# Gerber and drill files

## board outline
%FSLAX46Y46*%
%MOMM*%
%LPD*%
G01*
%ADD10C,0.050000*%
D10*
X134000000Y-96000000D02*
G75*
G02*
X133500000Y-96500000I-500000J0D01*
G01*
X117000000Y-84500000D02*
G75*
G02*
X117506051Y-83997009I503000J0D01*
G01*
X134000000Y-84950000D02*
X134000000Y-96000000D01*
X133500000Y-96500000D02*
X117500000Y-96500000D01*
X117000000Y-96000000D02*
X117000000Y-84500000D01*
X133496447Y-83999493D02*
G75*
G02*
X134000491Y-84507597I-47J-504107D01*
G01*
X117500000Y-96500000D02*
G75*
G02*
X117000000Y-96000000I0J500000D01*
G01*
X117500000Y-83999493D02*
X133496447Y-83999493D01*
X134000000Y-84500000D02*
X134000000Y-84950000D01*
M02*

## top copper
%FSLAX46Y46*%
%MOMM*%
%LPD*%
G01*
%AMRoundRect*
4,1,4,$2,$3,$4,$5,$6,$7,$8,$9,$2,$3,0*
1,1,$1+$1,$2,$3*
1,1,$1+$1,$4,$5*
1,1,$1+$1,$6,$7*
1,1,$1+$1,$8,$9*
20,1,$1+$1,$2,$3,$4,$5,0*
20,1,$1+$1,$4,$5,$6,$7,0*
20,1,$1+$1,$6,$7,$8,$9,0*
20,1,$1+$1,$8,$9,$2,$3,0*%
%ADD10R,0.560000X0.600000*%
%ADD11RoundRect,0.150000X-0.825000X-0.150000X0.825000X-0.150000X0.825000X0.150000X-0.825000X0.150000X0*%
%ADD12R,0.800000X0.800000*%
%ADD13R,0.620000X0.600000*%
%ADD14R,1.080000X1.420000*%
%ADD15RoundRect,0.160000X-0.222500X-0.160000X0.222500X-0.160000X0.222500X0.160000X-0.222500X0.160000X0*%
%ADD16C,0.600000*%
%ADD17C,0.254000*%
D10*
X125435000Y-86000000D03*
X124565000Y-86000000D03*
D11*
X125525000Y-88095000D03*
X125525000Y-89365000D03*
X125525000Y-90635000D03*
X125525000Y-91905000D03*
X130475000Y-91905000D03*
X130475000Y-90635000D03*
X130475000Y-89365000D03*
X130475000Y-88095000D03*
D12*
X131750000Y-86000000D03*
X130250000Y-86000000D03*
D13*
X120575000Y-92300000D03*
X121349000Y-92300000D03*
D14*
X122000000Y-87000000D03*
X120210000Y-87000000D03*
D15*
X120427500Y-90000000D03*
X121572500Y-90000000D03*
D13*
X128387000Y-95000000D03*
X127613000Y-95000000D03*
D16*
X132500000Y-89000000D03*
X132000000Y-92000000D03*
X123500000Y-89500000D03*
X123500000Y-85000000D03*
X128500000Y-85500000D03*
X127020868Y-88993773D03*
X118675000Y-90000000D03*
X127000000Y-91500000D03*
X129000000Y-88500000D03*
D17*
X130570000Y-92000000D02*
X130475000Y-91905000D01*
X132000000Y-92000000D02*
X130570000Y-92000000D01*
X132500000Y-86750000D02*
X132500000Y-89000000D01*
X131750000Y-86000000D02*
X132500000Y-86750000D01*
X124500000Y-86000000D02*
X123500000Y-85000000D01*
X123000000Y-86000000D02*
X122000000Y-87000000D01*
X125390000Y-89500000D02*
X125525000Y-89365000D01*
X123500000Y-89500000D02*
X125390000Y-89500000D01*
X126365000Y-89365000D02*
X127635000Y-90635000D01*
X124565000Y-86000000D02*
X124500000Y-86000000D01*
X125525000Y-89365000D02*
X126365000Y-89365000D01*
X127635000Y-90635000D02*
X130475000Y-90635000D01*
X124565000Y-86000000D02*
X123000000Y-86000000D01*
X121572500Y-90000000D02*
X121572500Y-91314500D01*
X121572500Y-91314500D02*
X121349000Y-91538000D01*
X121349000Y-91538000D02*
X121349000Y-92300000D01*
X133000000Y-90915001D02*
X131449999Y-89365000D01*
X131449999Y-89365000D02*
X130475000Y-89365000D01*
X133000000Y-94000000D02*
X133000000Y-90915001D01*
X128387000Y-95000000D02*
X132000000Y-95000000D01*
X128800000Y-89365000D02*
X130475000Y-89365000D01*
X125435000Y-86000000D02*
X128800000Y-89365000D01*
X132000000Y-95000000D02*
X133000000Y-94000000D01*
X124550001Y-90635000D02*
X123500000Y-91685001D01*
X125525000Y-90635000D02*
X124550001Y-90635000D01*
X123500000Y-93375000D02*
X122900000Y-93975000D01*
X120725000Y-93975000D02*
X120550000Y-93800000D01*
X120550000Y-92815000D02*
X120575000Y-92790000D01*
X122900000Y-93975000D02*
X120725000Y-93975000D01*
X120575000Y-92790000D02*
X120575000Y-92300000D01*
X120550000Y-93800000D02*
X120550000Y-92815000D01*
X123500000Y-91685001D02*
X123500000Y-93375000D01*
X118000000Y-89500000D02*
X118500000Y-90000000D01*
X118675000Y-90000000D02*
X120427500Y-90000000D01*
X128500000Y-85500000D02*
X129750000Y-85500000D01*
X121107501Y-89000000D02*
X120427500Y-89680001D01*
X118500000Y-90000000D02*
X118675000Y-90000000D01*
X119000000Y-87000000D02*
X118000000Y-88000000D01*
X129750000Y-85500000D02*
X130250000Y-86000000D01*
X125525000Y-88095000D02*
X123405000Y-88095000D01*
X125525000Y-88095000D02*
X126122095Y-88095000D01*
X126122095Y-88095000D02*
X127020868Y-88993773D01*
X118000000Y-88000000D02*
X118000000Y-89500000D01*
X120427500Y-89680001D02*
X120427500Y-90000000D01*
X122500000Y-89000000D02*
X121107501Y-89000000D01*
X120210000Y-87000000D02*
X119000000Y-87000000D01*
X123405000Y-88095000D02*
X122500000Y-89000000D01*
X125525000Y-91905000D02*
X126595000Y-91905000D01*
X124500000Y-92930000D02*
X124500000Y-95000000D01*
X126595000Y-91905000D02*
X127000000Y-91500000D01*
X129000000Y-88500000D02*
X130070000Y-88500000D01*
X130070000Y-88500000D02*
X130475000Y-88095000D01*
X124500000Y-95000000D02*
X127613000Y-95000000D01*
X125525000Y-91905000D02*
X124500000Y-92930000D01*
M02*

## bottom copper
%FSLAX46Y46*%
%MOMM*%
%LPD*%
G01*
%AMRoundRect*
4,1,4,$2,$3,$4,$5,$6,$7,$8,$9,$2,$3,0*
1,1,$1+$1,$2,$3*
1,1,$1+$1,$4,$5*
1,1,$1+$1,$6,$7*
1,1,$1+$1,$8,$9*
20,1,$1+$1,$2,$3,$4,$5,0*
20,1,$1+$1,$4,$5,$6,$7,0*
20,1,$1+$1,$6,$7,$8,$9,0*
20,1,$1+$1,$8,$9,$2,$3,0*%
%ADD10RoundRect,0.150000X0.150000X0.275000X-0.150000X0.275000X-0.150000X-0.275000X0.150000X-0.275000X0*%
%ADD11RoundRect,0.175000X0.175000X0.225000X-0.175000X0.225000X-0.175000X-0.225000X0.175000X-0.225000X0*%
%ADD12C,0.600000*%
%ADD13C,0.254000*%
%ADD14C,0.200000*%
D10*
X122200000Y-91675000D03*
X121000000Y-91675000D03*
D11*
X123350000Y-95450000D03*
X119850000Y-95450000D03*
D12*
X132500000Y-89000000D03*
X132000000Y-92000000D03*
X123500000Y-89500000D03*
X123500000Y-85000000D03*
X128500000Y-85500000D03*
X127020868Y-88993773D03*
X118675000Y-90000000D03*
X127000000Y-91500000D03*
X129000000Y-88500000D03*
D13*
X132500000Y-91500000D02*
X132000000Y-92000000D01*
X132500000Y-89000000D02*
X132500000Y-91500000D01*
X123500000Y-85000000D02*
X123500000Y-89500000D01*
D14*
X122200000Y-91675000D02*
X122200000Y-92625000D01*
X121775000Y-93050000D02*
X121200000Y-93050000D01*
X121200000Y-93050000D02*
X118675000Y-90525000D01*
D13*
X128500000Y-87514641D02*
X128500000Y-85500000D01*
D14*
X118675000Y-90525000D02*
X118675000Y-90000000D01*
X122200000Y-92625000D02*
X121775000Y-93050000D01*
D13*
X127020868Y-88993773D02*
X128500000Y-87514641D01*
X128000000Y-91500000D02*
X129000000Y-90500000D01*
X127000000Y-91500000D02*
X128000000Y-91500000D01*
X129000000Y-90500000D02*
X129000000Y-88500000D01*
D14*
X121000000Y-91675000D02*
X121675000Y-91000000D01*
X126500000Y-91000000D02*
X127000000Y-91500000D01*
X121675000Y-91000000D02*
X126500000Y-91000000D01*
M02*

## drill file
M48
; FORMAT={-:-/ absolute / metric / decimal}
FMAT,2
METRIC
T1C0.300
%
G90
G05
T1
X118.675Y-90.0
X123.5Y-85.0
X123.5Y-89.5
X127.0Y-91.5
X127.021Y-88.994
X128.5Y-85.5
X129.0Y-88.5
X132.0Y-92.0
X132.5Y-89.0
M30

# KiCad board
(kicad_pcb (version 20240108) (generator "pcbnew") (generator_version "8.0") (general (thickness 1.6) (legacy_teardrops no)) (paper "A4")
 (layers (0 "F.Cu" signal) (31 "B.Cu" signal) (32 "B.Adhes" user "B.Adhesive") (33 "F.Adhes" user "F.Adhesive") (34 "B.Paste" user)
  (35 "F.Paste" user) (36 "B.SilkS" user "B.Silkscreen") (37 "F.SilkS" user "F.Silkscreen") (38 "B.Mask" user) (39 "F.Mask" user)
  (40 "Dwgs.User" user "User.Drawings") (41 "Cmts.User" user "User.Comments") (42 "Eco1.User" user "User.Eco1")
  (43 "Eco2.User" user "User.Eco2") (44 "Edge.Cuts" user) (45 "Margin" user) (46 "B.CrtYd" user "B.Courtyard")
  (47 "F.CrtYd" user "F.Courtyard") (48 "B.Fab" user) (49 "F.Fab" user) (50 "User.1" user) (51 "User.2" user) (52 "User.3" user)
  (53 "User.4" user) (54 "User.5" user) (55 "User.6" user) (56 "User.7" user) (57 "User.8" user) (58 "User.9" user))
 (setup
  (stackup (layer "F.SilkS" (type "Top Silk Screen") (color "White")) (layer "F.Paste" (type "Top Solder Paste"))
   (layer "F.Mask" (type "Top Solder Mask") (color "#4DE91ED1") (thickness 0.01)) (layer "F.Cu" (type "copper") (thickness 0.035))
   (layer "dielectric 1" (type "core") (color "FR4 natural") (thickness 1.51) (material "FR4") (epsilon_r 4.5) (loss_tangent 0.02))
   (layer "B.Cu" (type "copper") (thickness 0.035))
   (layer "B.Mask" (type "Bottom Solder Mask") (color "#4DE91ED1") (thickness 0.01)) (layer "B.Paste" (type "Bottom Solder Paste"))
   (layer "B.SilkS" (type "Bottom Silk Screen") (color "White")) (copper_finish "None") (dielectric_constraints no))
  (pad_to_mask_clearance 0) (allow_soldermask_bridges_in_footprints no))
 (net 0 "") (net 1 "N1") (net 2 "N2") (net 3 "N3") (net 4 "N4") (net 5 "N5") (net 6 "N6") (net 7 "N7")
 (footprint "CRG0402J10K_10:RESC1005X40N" (layer "F.Cu") (at 125 86 180)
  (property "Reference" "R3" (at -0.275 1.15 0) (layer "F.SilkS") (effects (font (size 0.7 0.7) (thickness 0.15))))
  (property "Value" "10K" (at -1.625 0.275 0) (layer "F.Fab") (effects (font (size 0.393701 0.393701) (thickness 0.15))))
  (pad "1" smd rect (at -0.435 0 180) (size 0.56 0.6) (layers "F.Cu" "F.Paste" "F.Mask") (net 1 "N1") (solder_mask_margin 0.102))
  (pad "2" smd rect (at 0.435 0 180) (size 0.56 0.6) (layers "F.Cu" "F.Paste" "F.Mask") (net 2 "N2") (solder_mask_margin 0.102)))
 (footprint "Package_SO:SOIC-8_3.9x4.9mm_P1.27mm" (layer "F.Cu") (at 128 90)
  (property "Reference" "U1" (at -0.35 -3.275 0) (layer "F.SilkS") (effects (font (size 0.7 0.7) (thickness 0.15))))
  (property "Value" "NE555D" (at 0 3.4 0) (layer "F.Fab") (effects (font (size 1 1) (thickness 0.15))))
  (pad "1" smd roundrect (at -2.475 -1.905) (size 1.95 0.6) (layers "F.Cu" "F.Paste" "F.Mask") (roundrect_rratio 0.25) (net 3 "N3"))
  (pad "2" smd roundrect (at -2.475 -0.635) (size 1.95 0.6) (layers "F.Cu" "F.Paste" "F.Mask") (roundrect_rratio 0.25) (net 2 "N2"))
  (pad "3" smd roundrect (at -2.475 0.635) (size 1.95 0.6) (layers "F.Cu" "F.Paste" "F.Mask") (roundrect_rratio 0.25) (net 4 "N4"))
  (pad "4" smd roundrect (at -2.475 1.905) (size 1.95 0.6) (layers "F.Cu" "F.Paste" "F.Mask") (roundrect_rratio 0.25) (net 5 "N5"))
  (pad "5" smd roundrect (at 2.475 1.905) (size 1.95 0.6) (layers "F.Cu" "F.Paste" "F.Mask") (roundrect_rratio 0.25) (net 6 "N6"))
  (pad "6" smd roundrect (at 2.475 0.635) (size 1.95 0.6) (layers "F.Cu" "F.Paste" "F.Mask") (roundrect_rratio 0.25) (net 2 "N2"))
  (pad "7" smd roundrect (at 2.475 -0.635) (size 1.95 0.6) (layers "F.Cu" "F.Paste" "F.Mask") (roundrect_rratio 0.25) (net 1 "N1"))
  (pad "8" smd roundrect (at 2.475 -1.905) (size 1.95 0.6) (layers "F.Cu" "F.Paste" "F.Mask") (roundrect_rratio 0.25) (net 5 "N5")))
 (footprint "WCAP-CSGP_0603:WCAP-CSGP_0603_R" (layer "F.Cu") (at 131 86 180)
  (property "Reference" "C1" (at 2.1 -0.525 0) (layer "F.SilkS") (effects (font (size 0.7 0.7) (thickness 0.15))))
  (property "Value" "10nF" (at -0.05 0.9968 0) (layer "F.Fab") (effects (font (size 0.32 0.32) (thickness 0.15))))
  (pad "1" smd rect (at -0.75 0 180) (size 0.8 0.8) (layers "F.Cu" "F.Paste" "F.Mask") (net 6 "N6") (solder_mask_margin 0.102))
  (pad "2" smd rect (at 0.75 0 180) (size 0.8 0.8) (layers "F.Cu" "F.Paste" "F.Mask") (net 3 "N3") (solder_mask_margin 0.102)))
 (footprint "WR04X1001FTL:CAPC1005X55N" (layer "F.Cu") (at 120.962 92.3)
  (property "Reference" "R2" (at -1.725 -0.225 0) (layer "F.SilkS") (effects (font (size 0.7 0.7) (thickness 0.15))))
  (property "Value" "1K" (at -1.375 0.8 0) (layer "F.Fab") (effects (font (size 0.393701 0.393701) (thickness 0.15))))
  (pad "1" smd rect (at -0.387 0) (size 0.62 0.6) (layers "F.Cu" "F.Paste" "F.Mask") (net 4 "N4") (solder_mask_margin 0.05))
  (pad "2" smd rect (at 0.387 0) (size 0.62 0.6) (layers "F.Cu" "F.Paste" "F.Mask") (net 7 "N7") (solder_mask_margin 0.05)))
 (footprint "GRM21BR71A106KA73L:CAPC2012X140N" (layer "F.Cu") (at 121.105 87 180)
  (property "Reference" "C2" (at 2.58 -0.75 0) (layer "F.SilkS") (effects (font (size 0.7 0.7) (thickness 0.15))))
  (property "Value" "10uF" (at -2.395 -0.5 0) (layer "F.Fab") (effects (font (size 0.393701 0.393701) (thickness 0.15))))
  (pad "1" smd rect (at -0.895 0 180) (size 1.08 1.42) (layers "F.Cu" "F.Paste" "F.Mask") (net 2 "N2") (solder_mask_margin 0.102))
  (pad "2" smd rect (at 0.895 0 180) (size 1.08 1.42) (layers "F.Cu" "F.Paste" "F.Mask") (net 3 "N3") (solder_mask_margin 0.102)))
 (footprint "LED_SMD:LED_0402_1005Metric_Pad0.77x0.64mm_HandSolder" (layer "F.Cu") (at 121 90)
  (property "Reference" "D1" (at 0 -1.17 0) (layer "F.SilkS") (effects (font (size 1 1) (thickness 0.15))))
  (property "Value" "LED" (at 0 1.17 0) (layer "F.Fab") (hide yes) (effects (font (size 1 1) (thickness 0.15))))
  (pad "1" smd roundrect (at -0.5725 0) (size 0.765 0.64) (layers "F.Cu" "F.Paste" "F.Mask") (roundrect_rratio 0.25) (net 3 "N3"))
  (pad "2" smd roundrect (at 0.5725 0) (size 0.765 0.64) (layers "F.Cu" "F.Paste" "F.Mask") (roundrect_rratio 0.25) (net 7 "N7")))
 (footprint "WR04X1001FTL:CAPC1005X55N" (layer "F.Cu") (at 128 95 180)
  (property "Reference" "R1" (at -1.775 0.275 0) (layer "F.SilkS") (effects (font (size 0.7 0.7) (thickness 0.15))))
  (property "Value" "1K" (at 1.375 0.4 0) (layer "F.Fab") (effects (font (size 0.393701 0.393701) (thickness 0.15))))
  (pad "1" smd rect (at -0.387 0 180) (size 0.62 0.6) (layers "F.Cu" "F.Paste" "F.Mask") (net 1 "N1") (solder_mask_margin 0.05))
  (pad "2" smd rect (at 0.387 0 180) (size 0.62 0.6) (layers "F.Cu" "F.Paste" "F.Mask") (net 5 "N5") (solder_mask_margin 0.05)
   (teardrops (best_length_ratio 2) (max_length 1) (best_width_ratio 1) (max_width 2) (curve_points 0) (filter_ratio 0.9) (enabled no)
    (allow_two_segments yes) (prefer_zone_connections yes))))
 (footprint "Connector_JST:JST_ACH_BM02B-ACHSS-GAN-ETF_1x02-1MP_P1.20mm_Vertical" (layer "B.Cu") (at 121.6 93.55 180)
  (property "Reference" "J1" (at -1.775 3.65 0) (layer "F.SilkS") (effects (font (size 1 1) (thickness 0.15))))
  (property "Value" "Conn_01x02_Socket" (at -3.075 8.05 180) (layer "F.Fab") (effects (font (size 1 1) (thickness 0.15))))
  (pad "1" smd roundrect (at -0.6 1.875 180) (size 0.6 0.85) (layers "B.Cu" "B.Paste" "B.Mask") (roundrect_rratio 0.25) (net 3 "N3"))
  (pad "2" smd roundrect (at 0.6 1.875 180) (size 0.6 0.85) (layers "B.Cu" "B.Paste" "B.Mask") (roundrect_rratio 0.25) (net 5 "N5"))
  (pad "MP" smd roundrect (at -1.75 -1.9 180) (size 0.7 0.8) (layers "B.Cu" "B.Paste" "B.Mask") (roundrect_rratio 0.25))
  (pad "MP" smd roundrect (at 1.75 -1.9 180) (size 0.7 0.8) (layers "B.Cu" "B.Paste" "B.Mask") (roundrect_rratio 0.25)))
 (gr_arc (start 134 96) (mid 133.853553 96.353553) (end 133.5 96.5) (stroke (width 0.05) (type default)) (layer "Edge.Cuts"))
 (gr_arc (start 117 84.5) (mid 117.148404 84.143238) (end 117.506051 83.996979) (stroke (width 0.05) (type default)) (layer "Edge.Cuts"))
 (gr_line (start 134 84.95) (end 134 96) (stroke (width 0.05) (type default)) (layer "Edge.Cuts"))
 (gr_line (start 133.5 96.5) (end 117.5 96.5) (stroke (width 0.05) (type default)) (layer "Edge.Cuts"))
 (gr_line (start 117 96) (end 117 84.5) (stroke (width 0.05) (type default)) (layer "Edge.Cuts"))
 (gr_arc (start 133.496447 83.999493) (mid 133.854298 84.148562) (end 134.000491 84.507597) (stroke (width 0.05) (type default))
  (layer "Edge.Cuts"))
 (gr_arc (start 117.5 96.5) (mid 117.146447 96.353553) (end 117 96) (stroke (width 0.05) (type default)) (layer "Edge.Cuts"))
 (gr_line (start 117.5 83.999493) (end 133.496447 83.999493) (stroke (width 0.05) (type default)) (layer "Edge.Cuts"))
 (gr_line (start 134 84.5) (end 134 84.95) (stroke (width 0.05) (type default)) (layer "Edge.Cuts"))
 (segment (start 130.57 92) (end 130.475 91.905) (width 0.254) (layer "F.Cu") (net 6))
 (segment (start 132 92) (end 130.57 92) (width 0.254) (layer "F.Cu") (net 6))
 (segment (start 132.5 86.75) (end 132.5 89) (width 0.254) (layer "F.Cu") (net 6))
 (segment (start 131.75 86) (end 132.5 86.75) (width 0.254) (layer "F.Cu") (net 6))
 (via (at 132.5 89) (size 0.6) (drill 0.3) (layers "F.Cu" "B.Cu") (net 6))
 (via (at 132 92) (size 0.6) (drill 0.3) (layers "F.Cu" "B.Cu") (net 6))
 (segment (start 132.5 91.5) (end 132 92) (width 0.254) (layer "B.Cu") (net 6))
 (segment (start 132.5 89) (end 132.5 91.5) (width 0.254) (layer "B.Cu") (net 6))
 (segment (start 124.5 86) (end 123.5 85) (width 0.254) (layer "F.Cu") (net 2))
 (segment (start 123 86) (end 122 87) (width 0.254) (layer "F.Cu") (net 2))
 (segment (start 125.39 89.5) (end 125.525 89.365) (width 0.254) (layer "F.Cu") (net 2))
 (segment (start 123.5 89.5) (end 125.39 89.5) (width 0.254) (layer "F.Cu") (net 2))
 (segment (start 126.365 89.365) (end 127.635 90.635) (width 0.254) (layer "F.Cu") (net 2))
 (segment (start 124.565 86) (end 124.5 86) (width 0.254) (layer "F.Cu") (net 2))
 (segment (start 125.525 89.365) (end 126.365 89.365) (width 0.254) (layer "F.Cu") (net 2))
 (segment (start 127.635 90.635) (end 130.475 90.635) (width 0.254) (layer "F.Cu") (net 2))
 (segment (start 124.565 86) (end 123 86) (width 0.254) (layer "F.Cu") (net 2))
 (via (at 123.5 89.5) (size 0.6) (drill 0.3) (layers "F.Cu" "B.Cu") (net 2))
 (via (at 123.5 85) (size 0.6) (drill 0.3) (layers "F.Cu" "B.Cu") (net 2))
 (segment (start 123.5 85) (end 123.5 89.5) (width 0.254) (layer "B.Cu") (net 2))
 (segment (start 121.5725 90) (end 121.5725 91.3145) (width 0.254) (layer "F.Cu") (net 7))
 (segment (start 121.5725 91.3145) (end 121.349 91.538) (width 0.254) (layer "F.Cu") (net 7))
 (segment (start 121.349 91.538) (end 121.349 92.3) (width 0.254) (layer "F.Cu") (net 7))
 (segment (start 133 90.915001) (end 131.449999 89.365) (width 0.254) (layer "F.Cu") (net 1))
 (segment (start 131.449999 89.365) (end 130.475 89.365) (width 0.254) (layer "F.Cu") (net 1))
 (segment (start 133 94) (end 133 90.915001) (width 0.254) (layer "F.Cu") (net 1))
 (segment (start 128.387 95) (end 132 95) (width 0.254) (layer "F.Cu") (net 1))
 (segment (start 128.8 89.365) (end 130.475 89.365) (width 0.254) (layer "F.Cu") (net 1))
 (segment (start 125.435 86) (end 128.8 89.365) (width 0.254) (layer "F.Cu") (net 1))
 (segment (start 132 95) (end 133 94) (width 0.254) (layer "F.Cu") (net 1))
 (segment (start 124.550001 90.635) (end 123.5 91.685001) (width 0.254) (layer "F.Cu") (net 4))
 (segment (start 125.525 90.635) (end 124.550001 90.635) (width 0.254) (layer "F.Cu") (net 4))
 (segment (start 123.5 93.375) (end 122.9 93.975) (width 0.254) (layer "F.Cu") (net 4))
 (segment (start 120.725 93.975) (end 120.55 93.8) (width 0.254) (layer "F.Cu") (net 4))
 (segment (start 120.55 92.815) (end 120.575 92.79) (width 0.254) (layer "F.Cu") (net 4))
 (segment (start 122.9 93.975) (end 120.725 93.975) (width 0.254) (layer "F.Cu") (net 4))
 (segment (start 120.575 92.79) (end 120.575 92.3) (width 0.254) (layer "F.Cu") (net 4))
 (segment (start 120.55 93.8) (end 120.55 92.815) (width 0.254) (layer "F.Cu") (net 4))
 (segment (start 123.5 91.685001) (end 123.5 93.375) (width 0.254) (layer "F.Cu") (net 4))
 (segment (start 118 89.5) (end 118.5 90) (width 0.254) (layer "F.Cu") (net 3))
 (segment (start 118.675 90) (end 120.4275 90) (width 0.254) (layer "F.Cu") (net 3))
 (segment (start 128.5 85.5) (end 129.75 85.5) (width 0.254) (layer "F.Cu") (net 3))
 (segment (start 121.107501 89) (end 120.4275 89.680001) (width 0.254) (layer "F.Cu") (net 3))
 (segment (start 118.5 90) (end 118.675 90) (width 0.254) (layer "F.Cu") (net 3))
 (segment (start 119 87) (end 118 88) (width 0.254) (layer "F.Cu") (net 3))
 (segment (start 129.75 85.5) (end 130.25 86) (width 0.254) (layer "F.Cu") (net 3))
 (segment (start 125.525 88.095) (end 123.405 88.095) (width 0.254) (layer "F.Cu") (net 3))
 (segment (start 125.525 88.095) (end 126.122095 88.095) (width 0.254) (layer "F.Cu") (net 3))
 (segment (start 126.122095 88.095) (end 127.020868 88.993773) (width 0.254) (layer "F.Cu") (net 3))
 (segment (start 118 88) (end 118 89.5) (width 0.254) (layer "F.Cu") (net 3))
 (segment (start 120.4275 89.680001) (end 120.4275 90) (width 0.254) (layer "F.Cu") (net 3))
 (segment (start 122.5 89) (end 121.107501 89) (width 0.254) (layer "F.Cu") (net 3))
 (segment (start 120.21 87) (end 119 87) (width 0.254) (layer "F.Cu") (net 3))
 (segment (start 123.405 88.095) (end 122.5 89) (width 0.254) (layer "F.Cu") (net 3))
 (via (at 128.5 85.5) (size 0.6) (drill 0.3) (layers "F.Cu" "B.Cu") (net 3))
 (via (at 127.020868 88.993773) (size 0.6) (drill 0.3) (layers "F.Cu" "B.Cu") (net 3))
 (via (at 118.675 90) (size 0.6) (drill 0.3) (layers "F.Cu" "B.Cu") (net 3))
 (segment (start 122.2 91.675) (end 122.2 92.625) (width 0.2) (layer "B.Cu") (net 3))
 (segment (start 121.775 93.05) (end 121.2 93.05) (width 0.2) (layer "B.Cu") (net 3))
 (segment (start 121.2 93.05) (end 118.675 90.525) (width 0.2) (layer "B.Cu") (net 3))
 (segment (start 128.5 87.514641) (end 128.5 85.5) (width 0.254) (layer "B.Cu") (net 3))
 (segment (start 118.675 90.525) (end 118.675 90) (width 0.2) (layer "B.Cu") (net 3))
 (segment (start 122.2 92.625) (end 121.775 93.05) (width 0.2) (layer "B.Cu") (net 3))
 (segment (start 127.020868 88.993773) (end 128.5 87.514641) (width 0.254) (layer "B.Cu") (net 3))
 (segment (start 125.525 91.905) (end 126.595 91.905) (width 0.254) (layer "F.Cu") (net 5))
 (segment (start 124.5 92.93) (end 124.5 95) (width 0.254) (layer "F.Cu") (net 5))
 (segment (start 126.595 91.905) (end 127 91.5) (width 0.254) (layer "F.Cu") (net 5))
 (segment (start 129 88.5) (end 130.07 88.5) (width 0.254) (layer "F.Cu") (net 5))
 (segment (start 130.07 88.5) (end 130.475 88.095) (width 0.254) (layer "F.Cu") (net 5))
 (segment (start 124.5 95) (end 127.613 95) (width 0.254) (layer "F.Cu") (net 5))
 (segment (start 125.525 91.905) (end 124.5 92.93) (width 0.254) (layer "F.Cu") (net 5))
 (via (at 127 91.5) (size 0.6) (drill 0.3) (layers "F.Cu" "B.Cu") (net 5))
 (via (at 129 88.5) (size 0.6) (drill 0.3) (layers "F.Cu" "B.Cu") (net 5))
 (segment (start 128 91.5) (end 129 90.5) (width 0.254) (layer "B.Cu") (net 5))
 (segment (start 127 91.5) (end 128 91.5) (width 0.254) (layer "B.Cu") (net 5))
 (segment (start 129 90.5) (end 129 88.5) (width 0.254) (layer "B.Cu") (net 5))
 (segment (start 121 91.675) (end 121.675 91) (width 0.2) (layer "B.Cu") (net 5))
 (segment (start 126.5 91) (end 127 91.5) (width 0.2) (layer "B.Cu") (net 5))
 (segment (start 121.675 91) (end 126.5 91) (width 0.2) (layer "B.Cu") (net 5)))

